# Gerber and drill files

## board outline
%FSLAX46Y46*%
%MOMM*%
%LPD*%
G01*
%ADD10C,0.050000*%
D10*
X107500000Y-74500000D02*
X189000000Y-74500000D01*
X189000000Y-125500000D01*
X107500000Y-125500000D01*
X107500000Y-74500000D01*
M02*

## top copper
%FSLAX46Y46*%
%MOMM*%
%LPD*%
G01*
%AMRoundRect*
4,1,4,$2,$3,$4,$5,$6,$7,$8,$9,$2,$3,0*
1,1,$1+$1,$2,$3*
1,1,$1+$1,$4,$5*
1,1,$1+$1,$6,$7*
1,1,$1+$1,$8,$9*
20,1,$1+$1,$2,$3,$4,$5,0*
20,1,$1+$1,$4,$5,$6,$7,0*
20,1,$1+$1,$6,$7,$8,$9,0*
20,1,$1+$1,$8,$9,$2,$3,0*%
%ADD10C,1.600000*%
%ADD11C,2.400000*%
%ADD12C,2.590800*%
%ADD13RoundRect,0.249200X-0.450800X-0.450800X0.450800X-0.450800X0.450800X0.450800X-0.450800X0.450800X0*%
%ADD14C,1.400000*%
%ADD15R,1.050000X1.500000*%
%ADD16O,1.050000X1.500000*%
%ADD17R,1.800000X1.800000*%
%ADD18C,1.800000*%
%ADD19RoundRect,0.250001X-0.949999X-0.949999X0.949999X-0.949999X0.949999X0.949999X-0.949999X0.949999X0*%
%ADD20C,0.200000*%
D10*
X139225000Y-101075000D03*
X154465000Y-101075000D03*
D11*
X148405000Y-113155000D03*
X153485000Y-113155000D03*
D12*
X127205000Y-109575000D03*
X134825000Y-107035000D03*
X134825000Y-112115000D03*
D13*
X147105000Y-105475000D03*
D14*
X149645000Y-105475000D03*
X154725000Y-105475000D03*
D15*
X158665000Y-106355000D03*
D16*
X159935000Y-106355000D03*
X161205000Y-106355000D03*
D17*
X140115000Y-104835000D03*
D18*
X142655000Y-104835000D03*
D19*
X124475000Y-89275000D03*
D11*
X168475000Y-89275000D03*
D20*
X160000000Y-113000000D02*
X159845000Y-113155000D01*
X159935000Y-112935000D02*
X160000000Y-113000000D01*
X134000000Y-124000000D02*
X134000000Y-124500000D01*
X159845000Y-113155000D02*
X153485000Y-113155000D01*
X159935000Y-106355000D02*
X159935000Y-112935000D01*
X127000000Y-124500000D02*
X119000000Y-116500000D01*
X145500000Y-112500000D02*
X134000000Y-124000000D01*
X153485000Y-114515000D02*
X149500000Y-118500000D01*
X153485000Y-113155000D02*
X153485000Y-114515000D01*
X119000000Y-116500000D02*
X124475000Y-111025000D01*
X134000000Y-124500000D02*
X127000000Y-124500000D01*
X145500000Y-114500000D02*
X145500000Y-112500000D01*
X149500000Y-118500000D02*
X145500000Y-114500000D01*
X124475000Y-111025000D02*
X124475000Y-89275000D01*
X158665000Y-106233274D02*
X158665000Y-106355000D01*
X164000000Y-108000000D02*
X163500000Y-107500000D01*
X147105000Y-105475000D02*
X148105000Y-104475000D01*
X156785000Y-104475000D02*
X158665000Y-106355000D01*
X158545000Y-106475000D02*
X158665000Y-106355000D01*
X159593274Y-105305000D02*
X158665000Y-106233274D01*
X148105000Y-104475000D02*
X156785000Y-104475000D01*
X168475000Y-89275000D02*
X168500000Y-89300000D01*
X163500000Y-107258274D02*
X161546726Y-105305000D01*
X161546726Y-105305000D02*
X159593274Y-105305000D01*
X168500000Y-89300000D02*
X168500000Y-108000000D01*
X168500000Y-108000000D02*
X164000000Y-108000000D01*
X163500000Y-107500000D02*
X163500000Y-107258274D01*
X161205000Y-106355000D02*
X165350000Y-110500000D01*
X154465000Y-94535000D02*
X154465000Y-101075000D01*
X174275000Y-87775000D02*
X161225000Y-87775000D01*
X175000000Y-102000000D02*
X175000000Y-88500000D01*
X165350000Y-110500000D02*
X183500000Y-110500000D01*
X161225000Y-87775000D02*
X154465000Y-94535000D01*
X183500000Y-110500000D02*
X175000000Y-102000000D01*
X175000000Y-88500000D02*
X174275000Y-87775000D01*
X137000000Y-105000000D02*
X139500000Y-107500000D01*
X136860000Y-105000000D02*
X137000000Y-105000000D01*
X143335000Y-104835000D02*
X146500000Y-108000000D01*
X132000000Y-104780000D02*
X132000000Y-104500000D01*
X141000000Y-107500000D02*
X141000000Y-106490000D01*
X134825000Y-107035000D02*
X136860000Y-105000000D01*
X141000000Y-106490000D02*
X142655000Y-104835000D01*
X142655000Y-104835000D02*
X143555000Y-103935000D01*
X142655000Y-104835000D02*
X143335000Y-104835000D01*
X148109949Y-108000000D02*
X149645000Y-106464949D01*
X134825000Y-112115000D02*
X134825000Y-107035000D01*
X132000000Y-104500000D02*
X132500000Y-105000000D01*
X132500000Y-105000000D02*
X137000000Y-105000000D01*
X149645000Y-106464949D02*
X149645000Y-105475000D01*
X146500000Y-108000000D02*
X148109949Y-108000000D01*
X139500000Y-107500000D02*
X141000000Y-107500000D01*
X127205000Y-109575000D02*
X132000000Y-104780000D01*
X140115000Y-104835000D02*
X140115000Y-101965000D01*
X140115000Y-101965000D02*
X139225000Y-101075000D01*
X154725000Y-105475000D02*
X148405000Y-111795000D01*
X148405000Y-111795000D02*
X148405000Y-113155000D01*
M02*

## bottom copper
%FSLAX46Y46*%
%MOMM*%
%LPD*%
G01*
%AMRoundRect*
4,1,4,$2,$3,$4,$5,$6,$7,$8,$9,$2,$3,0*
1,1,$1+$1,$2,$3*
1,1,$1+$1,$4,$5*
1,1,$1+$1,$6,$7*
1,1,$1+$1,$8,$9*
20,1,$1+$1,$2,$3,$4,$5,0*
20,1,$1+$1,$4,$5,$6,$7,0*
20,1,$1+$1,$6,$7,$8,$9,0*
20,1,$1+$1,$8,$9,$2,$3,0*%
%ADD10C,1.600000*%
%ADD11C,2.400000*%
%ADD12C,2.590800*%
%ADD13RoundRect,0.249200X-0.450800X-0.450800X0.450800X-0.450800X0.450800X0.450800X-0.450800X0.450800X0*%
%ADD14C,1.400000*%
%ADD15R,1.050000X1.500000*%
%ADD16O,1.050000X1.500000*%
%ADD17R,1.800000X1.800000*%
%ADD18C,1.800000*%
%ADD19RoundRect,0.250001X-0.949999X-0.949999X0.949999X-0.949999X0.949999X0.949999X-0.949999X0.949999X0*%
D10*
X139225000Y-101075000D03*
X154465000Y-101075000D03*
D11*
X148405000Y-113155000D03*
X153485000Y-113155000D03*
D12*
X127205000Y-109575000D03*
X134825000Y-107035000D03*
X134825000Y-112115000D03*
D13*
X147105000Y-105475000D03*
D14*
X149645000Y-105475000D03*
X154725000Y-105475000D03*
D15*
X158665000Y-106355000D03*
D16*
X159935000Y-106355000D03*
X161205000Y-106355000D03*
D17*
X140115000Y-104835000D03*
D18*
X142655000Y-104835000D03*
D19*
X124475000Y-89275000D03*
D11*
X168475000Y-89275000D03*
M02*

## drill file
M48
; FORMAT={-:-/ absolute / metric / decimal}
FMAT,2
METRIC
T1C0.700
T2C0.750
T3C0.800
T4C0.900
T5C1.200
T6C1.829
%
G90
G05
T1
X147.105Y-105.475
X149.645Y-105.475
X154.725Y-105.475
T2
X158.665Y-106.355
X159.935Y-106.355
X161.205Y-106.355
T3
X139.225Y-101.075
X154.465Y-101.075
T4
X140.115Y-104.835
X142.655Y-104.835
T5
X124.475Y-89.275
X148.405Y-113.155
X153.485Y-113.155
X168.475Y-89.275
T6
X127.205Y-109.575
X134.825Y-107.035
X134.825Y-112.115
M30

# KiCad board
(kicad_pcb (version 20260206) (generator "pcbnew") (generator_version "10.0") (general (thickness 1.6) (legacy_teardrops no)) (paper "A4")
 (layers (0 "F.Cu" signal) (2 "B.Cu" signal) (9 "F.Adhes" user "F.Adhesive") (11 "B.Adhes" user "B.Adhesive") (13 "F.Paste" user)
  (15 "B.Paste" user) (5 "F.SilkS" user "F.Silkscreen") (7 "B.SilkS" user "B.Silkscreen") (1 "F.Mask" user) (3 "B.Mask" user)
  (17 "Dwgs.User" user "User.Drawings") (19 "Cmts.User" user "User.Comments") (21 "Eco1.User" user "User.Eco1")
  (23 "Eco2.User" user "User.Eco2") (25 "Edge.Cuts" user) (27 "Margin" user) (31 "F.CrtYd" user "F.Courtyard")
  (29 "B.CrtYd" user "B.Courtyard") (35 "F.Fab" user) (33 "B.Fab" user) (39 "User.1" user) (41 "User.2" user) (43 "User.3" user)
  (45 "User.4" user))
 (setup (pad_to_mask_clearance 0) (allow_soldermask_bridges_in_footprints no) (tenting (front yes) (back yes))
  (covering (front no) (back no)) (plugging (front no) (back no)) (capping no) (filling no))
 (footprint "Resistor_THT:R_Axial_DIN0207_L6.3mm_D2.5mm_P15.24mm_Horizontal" (layer "F.Cu") (at 139.225 101.075)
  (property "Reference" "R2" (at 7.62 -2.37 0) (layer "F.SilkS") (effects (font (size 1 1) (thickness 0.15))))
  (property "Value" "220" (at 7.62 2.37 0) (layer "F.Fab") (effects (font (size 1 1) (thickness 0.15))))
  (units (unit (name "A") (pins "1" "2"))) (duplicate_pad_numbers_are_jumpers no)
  (pad "1" thru_hole circle (at 0 0) (size 1.6 1.6) (drill 0.8) (layers "*.Cu" "*.Mask") (remove_unused_layers no) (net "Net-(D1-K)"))
  (pad "2" thru_hole circle (at 15.24 0) (size 1.6 1.6) (drill 0.8) (layers "*.Cu" "*.Mask") (remove_unused_layers no) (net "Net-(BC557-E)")))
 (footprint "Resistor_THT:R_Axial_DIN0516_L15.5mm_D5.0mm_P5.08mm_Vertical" (layer "F.Cu") (at 148.405 113.155)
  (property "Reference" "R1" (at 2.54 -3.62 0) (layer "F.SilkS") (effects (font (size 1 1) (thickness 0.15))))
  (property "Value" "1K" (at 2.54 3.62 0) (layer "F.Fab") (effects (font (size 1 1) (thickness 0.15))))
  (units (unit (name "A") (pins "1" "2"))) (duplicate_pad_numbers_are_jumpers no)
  (pad "1" thru_hole circle (at 0 0) (size 2.4 2.4) (drill 1.2) (layers "*.Cu" "*.Mask") (remove_unused_layers no) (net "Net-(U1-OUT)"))
  (pad "2" thru_hole circle (at 5.08 0) (size 2.4 2.4) (drill 1.2) (layers "*.Cu" "*.Mask") (remove_unused_layers no) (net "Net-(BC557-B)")))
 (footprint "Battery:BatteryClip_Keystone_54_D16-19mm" (layer "F.Cu") (at 127.205 109.575)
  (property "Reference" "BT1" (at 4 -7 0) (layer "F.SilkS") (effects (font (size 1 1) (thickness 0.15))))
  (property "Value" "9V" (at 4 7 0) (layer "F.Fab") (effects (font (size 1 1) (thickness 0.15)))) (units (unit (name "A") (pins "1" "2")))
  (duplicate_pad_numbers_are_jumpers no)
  (pad "1" thru_hole circle (at 0 0 180) (size 2.5908 2.5908) (drill 1.8288) (layers "*.Cu" "*.Mask") (remove_unused_layers no)
   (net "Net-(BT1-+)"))
  (pad "1" thru_hole circle (at 7.62 -2.54 180) (size 2.5908 2.5908) (drill 1.8288) (layers "*.Cu" "*.Mask") (remove_unused_layers no)
   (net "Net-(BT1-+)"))
  (pad "1" thru_hole circle (at 7.62 2.54 180) (size 2.5908 2.5908) (drill 1.8288) (layers "*.Cu" "*.Mask") (remove_unused_layers no)
   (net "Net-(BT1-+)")))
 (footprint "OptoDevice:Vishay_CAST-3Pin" (layer "F.Cu") (at 147.105 105.475)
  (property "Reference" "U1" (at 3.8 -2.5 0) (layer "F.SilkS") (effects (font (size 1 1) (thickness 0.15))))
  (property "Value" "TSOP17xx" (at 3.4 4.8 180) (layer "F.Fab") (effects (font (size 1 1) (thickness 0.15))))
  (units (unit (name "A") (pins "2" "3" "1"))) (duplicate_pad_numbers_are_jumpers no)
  (pad "1" thru_hole roundrect (at 0 0) (size 1.4 1.4) (drill 0.7) (layers "*.Cu" "*.Mask") (remove_unused_layers no)
   (roundrect_rratio 0.178) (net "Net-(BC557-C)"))
  (pad "2" thru_hole circle (at 2.54 0) (size 1.4 1.4) (drill 0.7) (layers "*.Cu" "*.Mask") (remove_unused_layers no) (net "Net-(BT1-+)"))
  (pad "3" thru_hole circle (at 7.62 0) (size 1.4 1.4) (drill 0.7) (layers "*.Cu" "*.Mask") (remove_unused_layers no) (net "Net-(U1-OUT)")))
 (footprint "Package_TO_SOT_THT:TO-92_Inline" (layer "F.Cu") (at 158.665 106.355)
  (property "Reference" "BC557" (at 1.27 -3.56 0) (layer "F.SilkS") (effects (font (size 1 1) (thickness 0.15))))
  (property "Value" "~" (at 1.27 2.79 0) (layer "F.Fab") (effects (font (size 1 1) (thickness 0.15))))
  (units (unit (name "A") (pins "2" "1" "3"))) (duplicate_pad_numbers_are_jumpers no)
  (pad "1" thru_hole rect (at 0 0) (size 1.05 1.5) (drill 0.75) (layers "*.Cu" "*.Mask") (remove_unused_layers no) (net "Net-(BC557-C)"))
  (pad "2" thru_hole oval (at 1.27 0) (size 1.05 1.5) (drill 0.75) (layers "*.Cu" "*.Mask") (remove_unused_layers no) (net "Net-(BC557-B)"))
  (pad "3" thru_hole oval (at 2.54 0) (size 1.05 1.5) (drill 0.75) (layers "*.Cu" "*.Mask") (remove_unused_layers no) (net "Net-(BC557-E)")))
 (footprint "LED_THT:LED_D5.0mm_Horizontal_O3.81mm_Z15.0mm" (layer "F.Cu") (at 140.115 104.835)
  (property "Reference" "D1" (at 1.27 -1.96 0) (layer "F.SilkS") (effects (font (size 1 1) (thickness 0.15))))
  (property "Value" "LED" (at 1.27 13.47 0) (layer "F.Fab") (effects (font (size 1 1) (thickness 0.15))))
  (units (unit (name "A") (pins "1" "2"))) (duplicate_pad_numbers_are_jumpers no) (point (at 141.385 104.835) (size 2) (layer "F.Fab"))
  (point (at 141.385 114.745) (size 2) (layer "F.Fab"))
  (pad "1" thru_hole rect (at 0 0) (size 1.8 1.8) (drill 0.9) (layers "*.Cu" "*.Mask") (remove_unused_layers no) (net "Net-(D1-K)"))
  (pad "2" thru_hole circle (at 2.54 0) (size 1.8 1.8) (drill 0.9) (layers "*.Cu" "*.Mask") (remove_unused_layers no) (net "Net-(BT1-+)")))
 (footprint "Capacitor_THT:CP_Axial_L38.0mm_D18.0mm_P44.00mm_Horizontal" (layer "F.Cu") (at 124.475 89.275)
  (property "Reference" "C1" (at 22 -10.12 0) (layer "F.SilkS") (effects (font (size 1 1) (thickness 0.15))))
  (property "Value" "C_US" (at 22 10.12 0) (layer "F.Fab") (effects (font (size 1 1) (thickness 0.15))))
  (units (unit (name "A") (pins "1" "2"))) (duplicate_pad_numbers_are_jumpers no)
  (pad "1" thru_hole roundrect (at 0 0) (size 2.4 2.4) (drill 1.2) (layers "*.Cu" "*.Mask") (remove_unused_layers no)
   (roundrect_rratio 0.104167) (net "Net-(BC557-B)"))
  (pad "2" thru_hole circle (at 44 0) (size 2.4 2.4) (drill 1.2) (layers "*.Cu" "*.Mask") (remove_unused_layers no) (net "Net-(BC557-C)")))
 (gr_rect (start 107.5 74.5) (end 189 125.5) (stroke (width 0.05) (type default)) (fill no) (layer "Edge.Cuts"))
 (segment (start 160 113) (end 159.845 113.155) (width 0.2) (layer "F.Cu") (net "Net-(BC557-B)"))
 (segment (start 159.935 112.935) (end 160 113) (width 0.2) (layer "F.Cu") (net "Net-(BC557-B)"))
 (segment (start 134 124) (end 134 124.5) (width 0.2) (layer "F.Cu") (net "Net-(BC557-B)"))
 (segment (start 159.845 113.155) (end 153.485 113.155) (width 0.2) (layer "F.Cu") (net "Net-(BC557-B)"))
 (segment (start 159.935 106.355) (end 159.935 112.935) (width 0.2) (layer "F.Cu") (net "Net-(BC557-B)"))
 (segment (start 127 124.5) (end 119 116.5) (width 0.2) (layer "F.Cu") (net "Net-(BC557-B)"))
 (segment (start 145.5 112.5) (end 134 124) (width 0.2) (layer "F.Cu") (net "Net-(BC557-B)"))
 (segment (start 153.485 114.515) (end 149.5 118.5) (width 0.2) (layer "F.Cu") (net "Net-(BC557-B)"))
 (segment (start 153.485 113.155) (end 153.485 114.515) (width 0.2) (layer "F.Cu") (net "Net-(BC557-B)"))
 (segment (start 119 116.5) (end 124.475 111.025) (width 0.2) (layer "F.Cu") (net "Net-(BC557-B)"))
 (segment (start 134 124.5) (end 127 124.5) (width 0.2) (layer "F.Cu") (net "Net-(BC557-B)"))
 (segment (start 145.5 114.5) (end 145.5 112.5) (width 0.2) (layer "F.Cu") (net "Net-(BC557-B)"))
 (segment (start 149.5 118.5) (end 145.5 114.5) (width 0.2) (layer "F.Cu") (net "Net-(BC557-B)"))
 (segment (start 124.475 111.025) (end 124.475 89.275) (width 0.2) (layer "F.Cu") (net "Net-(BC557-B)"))
 (segment (start 158.665 106.233274) (end 158.665 106.355) (width 0.2) (layer "F.Cu") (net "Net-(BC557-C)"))
 (segment (start 164 108) (end 163.5 107.5) (width 0.2) (layer "F.Cu") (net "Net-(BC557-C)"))
 (segment (start 147.105 105.475) (end 148.105 104.475) (width 0.2) (layer "F.Cu") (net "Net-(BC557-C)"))
 (segment (start 156.785 104.475) (end 158.665 106.355) (width 0.2) (layer "F.Cu") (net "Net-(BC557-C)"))
 (segment (start 158.545 106.475) (end 158.665 106.355) (width 0.2) (layer "F.Cu") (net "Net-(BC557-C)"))
 (segment (start 159.593274 105.305) (end 158.665 106.233274) (width 0.2) (layer "F.Cu") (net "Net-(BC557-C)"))
 (segment (start 148.105 104.475) (end 156.785 104.475) (width 0.2) (layer "F.Cu") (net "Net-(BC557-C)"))
 (segment (start 168.475 89.275) (end 168.5 89.3) (width 0.2) (layer "F.Cu") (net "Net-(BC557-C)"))
 (segment (start 163.5 107.258274) (end 161.546726 105.305) (width 0.2) (layer "F.Cu") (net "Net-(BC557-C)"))
 (segment (start 161.546726 105.305) (end 159.593274 105.305) (width 0.2) (layer "F.Cu") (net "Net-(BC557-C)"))
 (segment (start 168.5 89.3) (end 168.5 108) (width 0.2) (layer "F.Cu") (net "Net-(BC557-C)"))
 (segment (start 168.5 108) (end 164 108) (width 0.2) (layer "F.Cu") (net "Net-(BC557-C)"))
 (segment (start 163.5 107.5) (end 163.5 107.258274) (width 0.2) (layer "F.Cu") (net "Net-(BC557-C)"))
 (segment (start 161.205 106.355) (end 165.35 110.5) (width 0.2) (layer "F.Cu") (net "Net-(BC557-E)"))
 (segment (start 154.465 94.535) (end 154.465 101.075) (width 0.2) (layer "F.Cu") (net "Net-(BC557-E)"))
 (segment (start 174.275 87.775) (end 161.225 87.775) (width 0.2) (layer "F.Cu") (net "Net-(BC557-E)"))
 (segment (start 175 102) (end 175 88.5) (width 0.2) (layer "F.Cu") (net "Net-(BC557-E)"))
 (segment (start 165.35 110.5) (end 183.5 110.5) (width 0.2) (layer "F.Cu") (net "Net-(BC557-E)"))
 (segment (start 161.225 87.775) (end 154.465 94.535) (width 0.2) (layer "F.Cu") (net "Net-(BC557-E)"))
 (segment (start 183.5 110.5) (end 175 102) (width 0.2) (layer "F.Cu") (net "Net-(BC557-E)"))
 (segment (start 175 88.5) (end 174.275 87.775) (width 0.2) (layer "F.Cu") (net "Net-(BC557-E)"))
 (segment (start 137 105) (end 139.5 107.5) (width 0.2) (layer "F.Cu") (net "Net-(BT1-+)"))
 (segment (start 136.86 105) (end 137 105) (width 0.2) (layer "F.Cu") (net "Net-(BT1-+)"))
 (segment (start 143.335 104.835) (end 146.5 108) (width 0.2) (layer "F.Cu") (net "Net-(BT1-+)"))
 (segment (start 132 104.78) (end 132 104.5) (width 0.2) (layer "F.Cu") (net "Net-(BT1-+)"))
 (segment (start 141 107.5) (end 141 106.49) (width 0.2) (layer "F.Cu") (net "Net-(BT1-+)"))
 (segment (start 134.825 107.035) (end 136.86 105) (width 0.2) (layer "F.Cu") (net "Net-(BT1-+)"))
 (segment (start 141 106.49) (end 142.655 104.835) (width 0.2) (layer "F.Cu") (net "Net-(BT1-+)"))
 (segment (start 142.655 104.835) (end 143.555 103.935) (width 0.2) (layer "F.Cu") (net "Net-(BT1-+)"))
 (segment (start 142.655 104.835) (end 143.335 104.835) (width 0.2) (layer "F.Cu") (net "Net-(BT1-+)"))
 (segment (start 148.109949 108) (end 149.645 106.464949) (width 0.2) (layer "F.Cu") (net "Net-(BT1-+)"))
 (segment (start 134.825 112.115) (end 134.825 107.035) (width 0.2) (layer "F.Cu") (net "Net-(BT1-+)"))
 (segment (start 132 104.5) (end 132.5 105) (width 0.2) (layer "F.Cu") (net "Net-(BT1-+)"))
 (segment (start 132.5 105) (end 137 105) (width 0.2) (layer "F.Cu") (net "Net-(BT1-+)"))
 (segment (start 149.645 106.464949) (end 149.645 105.475) (width 0.2) (layer "F.Cu") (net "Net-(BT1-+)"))
 (segment (start 146.5 108) (end 148.109949 108) (width 0.2) (layer "F.Cu") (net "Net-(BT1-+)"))
 (segment (start 139.5 107.5) (end 141 107.5) (width 0.2) (layer "F.Cu") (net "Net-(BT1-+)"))
 (segment (start 127.205 109.575) (end 132 104.78) (width 0.2) (layer "F.Cu") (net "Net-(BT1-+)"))
 (segment (start 140.115 104.835) (end 140.115 101.965) (width 0.2) (layer "F.Cu") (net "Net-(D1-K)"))
 (segment (start 140.115 101.965) (end 139.225 101.075) (width 0.2) (layer "F.Cu") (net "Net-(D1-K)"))
 (segment (start 154.725 105.475) (end 148.405 111.795) (width 0.2) (layer "F.Cu") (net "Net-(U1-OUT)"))
 (segment (start 148.405 111.795) (end 148.405 113.155) (width 0.2) (layer "F.Cu") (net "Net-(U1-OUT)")))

